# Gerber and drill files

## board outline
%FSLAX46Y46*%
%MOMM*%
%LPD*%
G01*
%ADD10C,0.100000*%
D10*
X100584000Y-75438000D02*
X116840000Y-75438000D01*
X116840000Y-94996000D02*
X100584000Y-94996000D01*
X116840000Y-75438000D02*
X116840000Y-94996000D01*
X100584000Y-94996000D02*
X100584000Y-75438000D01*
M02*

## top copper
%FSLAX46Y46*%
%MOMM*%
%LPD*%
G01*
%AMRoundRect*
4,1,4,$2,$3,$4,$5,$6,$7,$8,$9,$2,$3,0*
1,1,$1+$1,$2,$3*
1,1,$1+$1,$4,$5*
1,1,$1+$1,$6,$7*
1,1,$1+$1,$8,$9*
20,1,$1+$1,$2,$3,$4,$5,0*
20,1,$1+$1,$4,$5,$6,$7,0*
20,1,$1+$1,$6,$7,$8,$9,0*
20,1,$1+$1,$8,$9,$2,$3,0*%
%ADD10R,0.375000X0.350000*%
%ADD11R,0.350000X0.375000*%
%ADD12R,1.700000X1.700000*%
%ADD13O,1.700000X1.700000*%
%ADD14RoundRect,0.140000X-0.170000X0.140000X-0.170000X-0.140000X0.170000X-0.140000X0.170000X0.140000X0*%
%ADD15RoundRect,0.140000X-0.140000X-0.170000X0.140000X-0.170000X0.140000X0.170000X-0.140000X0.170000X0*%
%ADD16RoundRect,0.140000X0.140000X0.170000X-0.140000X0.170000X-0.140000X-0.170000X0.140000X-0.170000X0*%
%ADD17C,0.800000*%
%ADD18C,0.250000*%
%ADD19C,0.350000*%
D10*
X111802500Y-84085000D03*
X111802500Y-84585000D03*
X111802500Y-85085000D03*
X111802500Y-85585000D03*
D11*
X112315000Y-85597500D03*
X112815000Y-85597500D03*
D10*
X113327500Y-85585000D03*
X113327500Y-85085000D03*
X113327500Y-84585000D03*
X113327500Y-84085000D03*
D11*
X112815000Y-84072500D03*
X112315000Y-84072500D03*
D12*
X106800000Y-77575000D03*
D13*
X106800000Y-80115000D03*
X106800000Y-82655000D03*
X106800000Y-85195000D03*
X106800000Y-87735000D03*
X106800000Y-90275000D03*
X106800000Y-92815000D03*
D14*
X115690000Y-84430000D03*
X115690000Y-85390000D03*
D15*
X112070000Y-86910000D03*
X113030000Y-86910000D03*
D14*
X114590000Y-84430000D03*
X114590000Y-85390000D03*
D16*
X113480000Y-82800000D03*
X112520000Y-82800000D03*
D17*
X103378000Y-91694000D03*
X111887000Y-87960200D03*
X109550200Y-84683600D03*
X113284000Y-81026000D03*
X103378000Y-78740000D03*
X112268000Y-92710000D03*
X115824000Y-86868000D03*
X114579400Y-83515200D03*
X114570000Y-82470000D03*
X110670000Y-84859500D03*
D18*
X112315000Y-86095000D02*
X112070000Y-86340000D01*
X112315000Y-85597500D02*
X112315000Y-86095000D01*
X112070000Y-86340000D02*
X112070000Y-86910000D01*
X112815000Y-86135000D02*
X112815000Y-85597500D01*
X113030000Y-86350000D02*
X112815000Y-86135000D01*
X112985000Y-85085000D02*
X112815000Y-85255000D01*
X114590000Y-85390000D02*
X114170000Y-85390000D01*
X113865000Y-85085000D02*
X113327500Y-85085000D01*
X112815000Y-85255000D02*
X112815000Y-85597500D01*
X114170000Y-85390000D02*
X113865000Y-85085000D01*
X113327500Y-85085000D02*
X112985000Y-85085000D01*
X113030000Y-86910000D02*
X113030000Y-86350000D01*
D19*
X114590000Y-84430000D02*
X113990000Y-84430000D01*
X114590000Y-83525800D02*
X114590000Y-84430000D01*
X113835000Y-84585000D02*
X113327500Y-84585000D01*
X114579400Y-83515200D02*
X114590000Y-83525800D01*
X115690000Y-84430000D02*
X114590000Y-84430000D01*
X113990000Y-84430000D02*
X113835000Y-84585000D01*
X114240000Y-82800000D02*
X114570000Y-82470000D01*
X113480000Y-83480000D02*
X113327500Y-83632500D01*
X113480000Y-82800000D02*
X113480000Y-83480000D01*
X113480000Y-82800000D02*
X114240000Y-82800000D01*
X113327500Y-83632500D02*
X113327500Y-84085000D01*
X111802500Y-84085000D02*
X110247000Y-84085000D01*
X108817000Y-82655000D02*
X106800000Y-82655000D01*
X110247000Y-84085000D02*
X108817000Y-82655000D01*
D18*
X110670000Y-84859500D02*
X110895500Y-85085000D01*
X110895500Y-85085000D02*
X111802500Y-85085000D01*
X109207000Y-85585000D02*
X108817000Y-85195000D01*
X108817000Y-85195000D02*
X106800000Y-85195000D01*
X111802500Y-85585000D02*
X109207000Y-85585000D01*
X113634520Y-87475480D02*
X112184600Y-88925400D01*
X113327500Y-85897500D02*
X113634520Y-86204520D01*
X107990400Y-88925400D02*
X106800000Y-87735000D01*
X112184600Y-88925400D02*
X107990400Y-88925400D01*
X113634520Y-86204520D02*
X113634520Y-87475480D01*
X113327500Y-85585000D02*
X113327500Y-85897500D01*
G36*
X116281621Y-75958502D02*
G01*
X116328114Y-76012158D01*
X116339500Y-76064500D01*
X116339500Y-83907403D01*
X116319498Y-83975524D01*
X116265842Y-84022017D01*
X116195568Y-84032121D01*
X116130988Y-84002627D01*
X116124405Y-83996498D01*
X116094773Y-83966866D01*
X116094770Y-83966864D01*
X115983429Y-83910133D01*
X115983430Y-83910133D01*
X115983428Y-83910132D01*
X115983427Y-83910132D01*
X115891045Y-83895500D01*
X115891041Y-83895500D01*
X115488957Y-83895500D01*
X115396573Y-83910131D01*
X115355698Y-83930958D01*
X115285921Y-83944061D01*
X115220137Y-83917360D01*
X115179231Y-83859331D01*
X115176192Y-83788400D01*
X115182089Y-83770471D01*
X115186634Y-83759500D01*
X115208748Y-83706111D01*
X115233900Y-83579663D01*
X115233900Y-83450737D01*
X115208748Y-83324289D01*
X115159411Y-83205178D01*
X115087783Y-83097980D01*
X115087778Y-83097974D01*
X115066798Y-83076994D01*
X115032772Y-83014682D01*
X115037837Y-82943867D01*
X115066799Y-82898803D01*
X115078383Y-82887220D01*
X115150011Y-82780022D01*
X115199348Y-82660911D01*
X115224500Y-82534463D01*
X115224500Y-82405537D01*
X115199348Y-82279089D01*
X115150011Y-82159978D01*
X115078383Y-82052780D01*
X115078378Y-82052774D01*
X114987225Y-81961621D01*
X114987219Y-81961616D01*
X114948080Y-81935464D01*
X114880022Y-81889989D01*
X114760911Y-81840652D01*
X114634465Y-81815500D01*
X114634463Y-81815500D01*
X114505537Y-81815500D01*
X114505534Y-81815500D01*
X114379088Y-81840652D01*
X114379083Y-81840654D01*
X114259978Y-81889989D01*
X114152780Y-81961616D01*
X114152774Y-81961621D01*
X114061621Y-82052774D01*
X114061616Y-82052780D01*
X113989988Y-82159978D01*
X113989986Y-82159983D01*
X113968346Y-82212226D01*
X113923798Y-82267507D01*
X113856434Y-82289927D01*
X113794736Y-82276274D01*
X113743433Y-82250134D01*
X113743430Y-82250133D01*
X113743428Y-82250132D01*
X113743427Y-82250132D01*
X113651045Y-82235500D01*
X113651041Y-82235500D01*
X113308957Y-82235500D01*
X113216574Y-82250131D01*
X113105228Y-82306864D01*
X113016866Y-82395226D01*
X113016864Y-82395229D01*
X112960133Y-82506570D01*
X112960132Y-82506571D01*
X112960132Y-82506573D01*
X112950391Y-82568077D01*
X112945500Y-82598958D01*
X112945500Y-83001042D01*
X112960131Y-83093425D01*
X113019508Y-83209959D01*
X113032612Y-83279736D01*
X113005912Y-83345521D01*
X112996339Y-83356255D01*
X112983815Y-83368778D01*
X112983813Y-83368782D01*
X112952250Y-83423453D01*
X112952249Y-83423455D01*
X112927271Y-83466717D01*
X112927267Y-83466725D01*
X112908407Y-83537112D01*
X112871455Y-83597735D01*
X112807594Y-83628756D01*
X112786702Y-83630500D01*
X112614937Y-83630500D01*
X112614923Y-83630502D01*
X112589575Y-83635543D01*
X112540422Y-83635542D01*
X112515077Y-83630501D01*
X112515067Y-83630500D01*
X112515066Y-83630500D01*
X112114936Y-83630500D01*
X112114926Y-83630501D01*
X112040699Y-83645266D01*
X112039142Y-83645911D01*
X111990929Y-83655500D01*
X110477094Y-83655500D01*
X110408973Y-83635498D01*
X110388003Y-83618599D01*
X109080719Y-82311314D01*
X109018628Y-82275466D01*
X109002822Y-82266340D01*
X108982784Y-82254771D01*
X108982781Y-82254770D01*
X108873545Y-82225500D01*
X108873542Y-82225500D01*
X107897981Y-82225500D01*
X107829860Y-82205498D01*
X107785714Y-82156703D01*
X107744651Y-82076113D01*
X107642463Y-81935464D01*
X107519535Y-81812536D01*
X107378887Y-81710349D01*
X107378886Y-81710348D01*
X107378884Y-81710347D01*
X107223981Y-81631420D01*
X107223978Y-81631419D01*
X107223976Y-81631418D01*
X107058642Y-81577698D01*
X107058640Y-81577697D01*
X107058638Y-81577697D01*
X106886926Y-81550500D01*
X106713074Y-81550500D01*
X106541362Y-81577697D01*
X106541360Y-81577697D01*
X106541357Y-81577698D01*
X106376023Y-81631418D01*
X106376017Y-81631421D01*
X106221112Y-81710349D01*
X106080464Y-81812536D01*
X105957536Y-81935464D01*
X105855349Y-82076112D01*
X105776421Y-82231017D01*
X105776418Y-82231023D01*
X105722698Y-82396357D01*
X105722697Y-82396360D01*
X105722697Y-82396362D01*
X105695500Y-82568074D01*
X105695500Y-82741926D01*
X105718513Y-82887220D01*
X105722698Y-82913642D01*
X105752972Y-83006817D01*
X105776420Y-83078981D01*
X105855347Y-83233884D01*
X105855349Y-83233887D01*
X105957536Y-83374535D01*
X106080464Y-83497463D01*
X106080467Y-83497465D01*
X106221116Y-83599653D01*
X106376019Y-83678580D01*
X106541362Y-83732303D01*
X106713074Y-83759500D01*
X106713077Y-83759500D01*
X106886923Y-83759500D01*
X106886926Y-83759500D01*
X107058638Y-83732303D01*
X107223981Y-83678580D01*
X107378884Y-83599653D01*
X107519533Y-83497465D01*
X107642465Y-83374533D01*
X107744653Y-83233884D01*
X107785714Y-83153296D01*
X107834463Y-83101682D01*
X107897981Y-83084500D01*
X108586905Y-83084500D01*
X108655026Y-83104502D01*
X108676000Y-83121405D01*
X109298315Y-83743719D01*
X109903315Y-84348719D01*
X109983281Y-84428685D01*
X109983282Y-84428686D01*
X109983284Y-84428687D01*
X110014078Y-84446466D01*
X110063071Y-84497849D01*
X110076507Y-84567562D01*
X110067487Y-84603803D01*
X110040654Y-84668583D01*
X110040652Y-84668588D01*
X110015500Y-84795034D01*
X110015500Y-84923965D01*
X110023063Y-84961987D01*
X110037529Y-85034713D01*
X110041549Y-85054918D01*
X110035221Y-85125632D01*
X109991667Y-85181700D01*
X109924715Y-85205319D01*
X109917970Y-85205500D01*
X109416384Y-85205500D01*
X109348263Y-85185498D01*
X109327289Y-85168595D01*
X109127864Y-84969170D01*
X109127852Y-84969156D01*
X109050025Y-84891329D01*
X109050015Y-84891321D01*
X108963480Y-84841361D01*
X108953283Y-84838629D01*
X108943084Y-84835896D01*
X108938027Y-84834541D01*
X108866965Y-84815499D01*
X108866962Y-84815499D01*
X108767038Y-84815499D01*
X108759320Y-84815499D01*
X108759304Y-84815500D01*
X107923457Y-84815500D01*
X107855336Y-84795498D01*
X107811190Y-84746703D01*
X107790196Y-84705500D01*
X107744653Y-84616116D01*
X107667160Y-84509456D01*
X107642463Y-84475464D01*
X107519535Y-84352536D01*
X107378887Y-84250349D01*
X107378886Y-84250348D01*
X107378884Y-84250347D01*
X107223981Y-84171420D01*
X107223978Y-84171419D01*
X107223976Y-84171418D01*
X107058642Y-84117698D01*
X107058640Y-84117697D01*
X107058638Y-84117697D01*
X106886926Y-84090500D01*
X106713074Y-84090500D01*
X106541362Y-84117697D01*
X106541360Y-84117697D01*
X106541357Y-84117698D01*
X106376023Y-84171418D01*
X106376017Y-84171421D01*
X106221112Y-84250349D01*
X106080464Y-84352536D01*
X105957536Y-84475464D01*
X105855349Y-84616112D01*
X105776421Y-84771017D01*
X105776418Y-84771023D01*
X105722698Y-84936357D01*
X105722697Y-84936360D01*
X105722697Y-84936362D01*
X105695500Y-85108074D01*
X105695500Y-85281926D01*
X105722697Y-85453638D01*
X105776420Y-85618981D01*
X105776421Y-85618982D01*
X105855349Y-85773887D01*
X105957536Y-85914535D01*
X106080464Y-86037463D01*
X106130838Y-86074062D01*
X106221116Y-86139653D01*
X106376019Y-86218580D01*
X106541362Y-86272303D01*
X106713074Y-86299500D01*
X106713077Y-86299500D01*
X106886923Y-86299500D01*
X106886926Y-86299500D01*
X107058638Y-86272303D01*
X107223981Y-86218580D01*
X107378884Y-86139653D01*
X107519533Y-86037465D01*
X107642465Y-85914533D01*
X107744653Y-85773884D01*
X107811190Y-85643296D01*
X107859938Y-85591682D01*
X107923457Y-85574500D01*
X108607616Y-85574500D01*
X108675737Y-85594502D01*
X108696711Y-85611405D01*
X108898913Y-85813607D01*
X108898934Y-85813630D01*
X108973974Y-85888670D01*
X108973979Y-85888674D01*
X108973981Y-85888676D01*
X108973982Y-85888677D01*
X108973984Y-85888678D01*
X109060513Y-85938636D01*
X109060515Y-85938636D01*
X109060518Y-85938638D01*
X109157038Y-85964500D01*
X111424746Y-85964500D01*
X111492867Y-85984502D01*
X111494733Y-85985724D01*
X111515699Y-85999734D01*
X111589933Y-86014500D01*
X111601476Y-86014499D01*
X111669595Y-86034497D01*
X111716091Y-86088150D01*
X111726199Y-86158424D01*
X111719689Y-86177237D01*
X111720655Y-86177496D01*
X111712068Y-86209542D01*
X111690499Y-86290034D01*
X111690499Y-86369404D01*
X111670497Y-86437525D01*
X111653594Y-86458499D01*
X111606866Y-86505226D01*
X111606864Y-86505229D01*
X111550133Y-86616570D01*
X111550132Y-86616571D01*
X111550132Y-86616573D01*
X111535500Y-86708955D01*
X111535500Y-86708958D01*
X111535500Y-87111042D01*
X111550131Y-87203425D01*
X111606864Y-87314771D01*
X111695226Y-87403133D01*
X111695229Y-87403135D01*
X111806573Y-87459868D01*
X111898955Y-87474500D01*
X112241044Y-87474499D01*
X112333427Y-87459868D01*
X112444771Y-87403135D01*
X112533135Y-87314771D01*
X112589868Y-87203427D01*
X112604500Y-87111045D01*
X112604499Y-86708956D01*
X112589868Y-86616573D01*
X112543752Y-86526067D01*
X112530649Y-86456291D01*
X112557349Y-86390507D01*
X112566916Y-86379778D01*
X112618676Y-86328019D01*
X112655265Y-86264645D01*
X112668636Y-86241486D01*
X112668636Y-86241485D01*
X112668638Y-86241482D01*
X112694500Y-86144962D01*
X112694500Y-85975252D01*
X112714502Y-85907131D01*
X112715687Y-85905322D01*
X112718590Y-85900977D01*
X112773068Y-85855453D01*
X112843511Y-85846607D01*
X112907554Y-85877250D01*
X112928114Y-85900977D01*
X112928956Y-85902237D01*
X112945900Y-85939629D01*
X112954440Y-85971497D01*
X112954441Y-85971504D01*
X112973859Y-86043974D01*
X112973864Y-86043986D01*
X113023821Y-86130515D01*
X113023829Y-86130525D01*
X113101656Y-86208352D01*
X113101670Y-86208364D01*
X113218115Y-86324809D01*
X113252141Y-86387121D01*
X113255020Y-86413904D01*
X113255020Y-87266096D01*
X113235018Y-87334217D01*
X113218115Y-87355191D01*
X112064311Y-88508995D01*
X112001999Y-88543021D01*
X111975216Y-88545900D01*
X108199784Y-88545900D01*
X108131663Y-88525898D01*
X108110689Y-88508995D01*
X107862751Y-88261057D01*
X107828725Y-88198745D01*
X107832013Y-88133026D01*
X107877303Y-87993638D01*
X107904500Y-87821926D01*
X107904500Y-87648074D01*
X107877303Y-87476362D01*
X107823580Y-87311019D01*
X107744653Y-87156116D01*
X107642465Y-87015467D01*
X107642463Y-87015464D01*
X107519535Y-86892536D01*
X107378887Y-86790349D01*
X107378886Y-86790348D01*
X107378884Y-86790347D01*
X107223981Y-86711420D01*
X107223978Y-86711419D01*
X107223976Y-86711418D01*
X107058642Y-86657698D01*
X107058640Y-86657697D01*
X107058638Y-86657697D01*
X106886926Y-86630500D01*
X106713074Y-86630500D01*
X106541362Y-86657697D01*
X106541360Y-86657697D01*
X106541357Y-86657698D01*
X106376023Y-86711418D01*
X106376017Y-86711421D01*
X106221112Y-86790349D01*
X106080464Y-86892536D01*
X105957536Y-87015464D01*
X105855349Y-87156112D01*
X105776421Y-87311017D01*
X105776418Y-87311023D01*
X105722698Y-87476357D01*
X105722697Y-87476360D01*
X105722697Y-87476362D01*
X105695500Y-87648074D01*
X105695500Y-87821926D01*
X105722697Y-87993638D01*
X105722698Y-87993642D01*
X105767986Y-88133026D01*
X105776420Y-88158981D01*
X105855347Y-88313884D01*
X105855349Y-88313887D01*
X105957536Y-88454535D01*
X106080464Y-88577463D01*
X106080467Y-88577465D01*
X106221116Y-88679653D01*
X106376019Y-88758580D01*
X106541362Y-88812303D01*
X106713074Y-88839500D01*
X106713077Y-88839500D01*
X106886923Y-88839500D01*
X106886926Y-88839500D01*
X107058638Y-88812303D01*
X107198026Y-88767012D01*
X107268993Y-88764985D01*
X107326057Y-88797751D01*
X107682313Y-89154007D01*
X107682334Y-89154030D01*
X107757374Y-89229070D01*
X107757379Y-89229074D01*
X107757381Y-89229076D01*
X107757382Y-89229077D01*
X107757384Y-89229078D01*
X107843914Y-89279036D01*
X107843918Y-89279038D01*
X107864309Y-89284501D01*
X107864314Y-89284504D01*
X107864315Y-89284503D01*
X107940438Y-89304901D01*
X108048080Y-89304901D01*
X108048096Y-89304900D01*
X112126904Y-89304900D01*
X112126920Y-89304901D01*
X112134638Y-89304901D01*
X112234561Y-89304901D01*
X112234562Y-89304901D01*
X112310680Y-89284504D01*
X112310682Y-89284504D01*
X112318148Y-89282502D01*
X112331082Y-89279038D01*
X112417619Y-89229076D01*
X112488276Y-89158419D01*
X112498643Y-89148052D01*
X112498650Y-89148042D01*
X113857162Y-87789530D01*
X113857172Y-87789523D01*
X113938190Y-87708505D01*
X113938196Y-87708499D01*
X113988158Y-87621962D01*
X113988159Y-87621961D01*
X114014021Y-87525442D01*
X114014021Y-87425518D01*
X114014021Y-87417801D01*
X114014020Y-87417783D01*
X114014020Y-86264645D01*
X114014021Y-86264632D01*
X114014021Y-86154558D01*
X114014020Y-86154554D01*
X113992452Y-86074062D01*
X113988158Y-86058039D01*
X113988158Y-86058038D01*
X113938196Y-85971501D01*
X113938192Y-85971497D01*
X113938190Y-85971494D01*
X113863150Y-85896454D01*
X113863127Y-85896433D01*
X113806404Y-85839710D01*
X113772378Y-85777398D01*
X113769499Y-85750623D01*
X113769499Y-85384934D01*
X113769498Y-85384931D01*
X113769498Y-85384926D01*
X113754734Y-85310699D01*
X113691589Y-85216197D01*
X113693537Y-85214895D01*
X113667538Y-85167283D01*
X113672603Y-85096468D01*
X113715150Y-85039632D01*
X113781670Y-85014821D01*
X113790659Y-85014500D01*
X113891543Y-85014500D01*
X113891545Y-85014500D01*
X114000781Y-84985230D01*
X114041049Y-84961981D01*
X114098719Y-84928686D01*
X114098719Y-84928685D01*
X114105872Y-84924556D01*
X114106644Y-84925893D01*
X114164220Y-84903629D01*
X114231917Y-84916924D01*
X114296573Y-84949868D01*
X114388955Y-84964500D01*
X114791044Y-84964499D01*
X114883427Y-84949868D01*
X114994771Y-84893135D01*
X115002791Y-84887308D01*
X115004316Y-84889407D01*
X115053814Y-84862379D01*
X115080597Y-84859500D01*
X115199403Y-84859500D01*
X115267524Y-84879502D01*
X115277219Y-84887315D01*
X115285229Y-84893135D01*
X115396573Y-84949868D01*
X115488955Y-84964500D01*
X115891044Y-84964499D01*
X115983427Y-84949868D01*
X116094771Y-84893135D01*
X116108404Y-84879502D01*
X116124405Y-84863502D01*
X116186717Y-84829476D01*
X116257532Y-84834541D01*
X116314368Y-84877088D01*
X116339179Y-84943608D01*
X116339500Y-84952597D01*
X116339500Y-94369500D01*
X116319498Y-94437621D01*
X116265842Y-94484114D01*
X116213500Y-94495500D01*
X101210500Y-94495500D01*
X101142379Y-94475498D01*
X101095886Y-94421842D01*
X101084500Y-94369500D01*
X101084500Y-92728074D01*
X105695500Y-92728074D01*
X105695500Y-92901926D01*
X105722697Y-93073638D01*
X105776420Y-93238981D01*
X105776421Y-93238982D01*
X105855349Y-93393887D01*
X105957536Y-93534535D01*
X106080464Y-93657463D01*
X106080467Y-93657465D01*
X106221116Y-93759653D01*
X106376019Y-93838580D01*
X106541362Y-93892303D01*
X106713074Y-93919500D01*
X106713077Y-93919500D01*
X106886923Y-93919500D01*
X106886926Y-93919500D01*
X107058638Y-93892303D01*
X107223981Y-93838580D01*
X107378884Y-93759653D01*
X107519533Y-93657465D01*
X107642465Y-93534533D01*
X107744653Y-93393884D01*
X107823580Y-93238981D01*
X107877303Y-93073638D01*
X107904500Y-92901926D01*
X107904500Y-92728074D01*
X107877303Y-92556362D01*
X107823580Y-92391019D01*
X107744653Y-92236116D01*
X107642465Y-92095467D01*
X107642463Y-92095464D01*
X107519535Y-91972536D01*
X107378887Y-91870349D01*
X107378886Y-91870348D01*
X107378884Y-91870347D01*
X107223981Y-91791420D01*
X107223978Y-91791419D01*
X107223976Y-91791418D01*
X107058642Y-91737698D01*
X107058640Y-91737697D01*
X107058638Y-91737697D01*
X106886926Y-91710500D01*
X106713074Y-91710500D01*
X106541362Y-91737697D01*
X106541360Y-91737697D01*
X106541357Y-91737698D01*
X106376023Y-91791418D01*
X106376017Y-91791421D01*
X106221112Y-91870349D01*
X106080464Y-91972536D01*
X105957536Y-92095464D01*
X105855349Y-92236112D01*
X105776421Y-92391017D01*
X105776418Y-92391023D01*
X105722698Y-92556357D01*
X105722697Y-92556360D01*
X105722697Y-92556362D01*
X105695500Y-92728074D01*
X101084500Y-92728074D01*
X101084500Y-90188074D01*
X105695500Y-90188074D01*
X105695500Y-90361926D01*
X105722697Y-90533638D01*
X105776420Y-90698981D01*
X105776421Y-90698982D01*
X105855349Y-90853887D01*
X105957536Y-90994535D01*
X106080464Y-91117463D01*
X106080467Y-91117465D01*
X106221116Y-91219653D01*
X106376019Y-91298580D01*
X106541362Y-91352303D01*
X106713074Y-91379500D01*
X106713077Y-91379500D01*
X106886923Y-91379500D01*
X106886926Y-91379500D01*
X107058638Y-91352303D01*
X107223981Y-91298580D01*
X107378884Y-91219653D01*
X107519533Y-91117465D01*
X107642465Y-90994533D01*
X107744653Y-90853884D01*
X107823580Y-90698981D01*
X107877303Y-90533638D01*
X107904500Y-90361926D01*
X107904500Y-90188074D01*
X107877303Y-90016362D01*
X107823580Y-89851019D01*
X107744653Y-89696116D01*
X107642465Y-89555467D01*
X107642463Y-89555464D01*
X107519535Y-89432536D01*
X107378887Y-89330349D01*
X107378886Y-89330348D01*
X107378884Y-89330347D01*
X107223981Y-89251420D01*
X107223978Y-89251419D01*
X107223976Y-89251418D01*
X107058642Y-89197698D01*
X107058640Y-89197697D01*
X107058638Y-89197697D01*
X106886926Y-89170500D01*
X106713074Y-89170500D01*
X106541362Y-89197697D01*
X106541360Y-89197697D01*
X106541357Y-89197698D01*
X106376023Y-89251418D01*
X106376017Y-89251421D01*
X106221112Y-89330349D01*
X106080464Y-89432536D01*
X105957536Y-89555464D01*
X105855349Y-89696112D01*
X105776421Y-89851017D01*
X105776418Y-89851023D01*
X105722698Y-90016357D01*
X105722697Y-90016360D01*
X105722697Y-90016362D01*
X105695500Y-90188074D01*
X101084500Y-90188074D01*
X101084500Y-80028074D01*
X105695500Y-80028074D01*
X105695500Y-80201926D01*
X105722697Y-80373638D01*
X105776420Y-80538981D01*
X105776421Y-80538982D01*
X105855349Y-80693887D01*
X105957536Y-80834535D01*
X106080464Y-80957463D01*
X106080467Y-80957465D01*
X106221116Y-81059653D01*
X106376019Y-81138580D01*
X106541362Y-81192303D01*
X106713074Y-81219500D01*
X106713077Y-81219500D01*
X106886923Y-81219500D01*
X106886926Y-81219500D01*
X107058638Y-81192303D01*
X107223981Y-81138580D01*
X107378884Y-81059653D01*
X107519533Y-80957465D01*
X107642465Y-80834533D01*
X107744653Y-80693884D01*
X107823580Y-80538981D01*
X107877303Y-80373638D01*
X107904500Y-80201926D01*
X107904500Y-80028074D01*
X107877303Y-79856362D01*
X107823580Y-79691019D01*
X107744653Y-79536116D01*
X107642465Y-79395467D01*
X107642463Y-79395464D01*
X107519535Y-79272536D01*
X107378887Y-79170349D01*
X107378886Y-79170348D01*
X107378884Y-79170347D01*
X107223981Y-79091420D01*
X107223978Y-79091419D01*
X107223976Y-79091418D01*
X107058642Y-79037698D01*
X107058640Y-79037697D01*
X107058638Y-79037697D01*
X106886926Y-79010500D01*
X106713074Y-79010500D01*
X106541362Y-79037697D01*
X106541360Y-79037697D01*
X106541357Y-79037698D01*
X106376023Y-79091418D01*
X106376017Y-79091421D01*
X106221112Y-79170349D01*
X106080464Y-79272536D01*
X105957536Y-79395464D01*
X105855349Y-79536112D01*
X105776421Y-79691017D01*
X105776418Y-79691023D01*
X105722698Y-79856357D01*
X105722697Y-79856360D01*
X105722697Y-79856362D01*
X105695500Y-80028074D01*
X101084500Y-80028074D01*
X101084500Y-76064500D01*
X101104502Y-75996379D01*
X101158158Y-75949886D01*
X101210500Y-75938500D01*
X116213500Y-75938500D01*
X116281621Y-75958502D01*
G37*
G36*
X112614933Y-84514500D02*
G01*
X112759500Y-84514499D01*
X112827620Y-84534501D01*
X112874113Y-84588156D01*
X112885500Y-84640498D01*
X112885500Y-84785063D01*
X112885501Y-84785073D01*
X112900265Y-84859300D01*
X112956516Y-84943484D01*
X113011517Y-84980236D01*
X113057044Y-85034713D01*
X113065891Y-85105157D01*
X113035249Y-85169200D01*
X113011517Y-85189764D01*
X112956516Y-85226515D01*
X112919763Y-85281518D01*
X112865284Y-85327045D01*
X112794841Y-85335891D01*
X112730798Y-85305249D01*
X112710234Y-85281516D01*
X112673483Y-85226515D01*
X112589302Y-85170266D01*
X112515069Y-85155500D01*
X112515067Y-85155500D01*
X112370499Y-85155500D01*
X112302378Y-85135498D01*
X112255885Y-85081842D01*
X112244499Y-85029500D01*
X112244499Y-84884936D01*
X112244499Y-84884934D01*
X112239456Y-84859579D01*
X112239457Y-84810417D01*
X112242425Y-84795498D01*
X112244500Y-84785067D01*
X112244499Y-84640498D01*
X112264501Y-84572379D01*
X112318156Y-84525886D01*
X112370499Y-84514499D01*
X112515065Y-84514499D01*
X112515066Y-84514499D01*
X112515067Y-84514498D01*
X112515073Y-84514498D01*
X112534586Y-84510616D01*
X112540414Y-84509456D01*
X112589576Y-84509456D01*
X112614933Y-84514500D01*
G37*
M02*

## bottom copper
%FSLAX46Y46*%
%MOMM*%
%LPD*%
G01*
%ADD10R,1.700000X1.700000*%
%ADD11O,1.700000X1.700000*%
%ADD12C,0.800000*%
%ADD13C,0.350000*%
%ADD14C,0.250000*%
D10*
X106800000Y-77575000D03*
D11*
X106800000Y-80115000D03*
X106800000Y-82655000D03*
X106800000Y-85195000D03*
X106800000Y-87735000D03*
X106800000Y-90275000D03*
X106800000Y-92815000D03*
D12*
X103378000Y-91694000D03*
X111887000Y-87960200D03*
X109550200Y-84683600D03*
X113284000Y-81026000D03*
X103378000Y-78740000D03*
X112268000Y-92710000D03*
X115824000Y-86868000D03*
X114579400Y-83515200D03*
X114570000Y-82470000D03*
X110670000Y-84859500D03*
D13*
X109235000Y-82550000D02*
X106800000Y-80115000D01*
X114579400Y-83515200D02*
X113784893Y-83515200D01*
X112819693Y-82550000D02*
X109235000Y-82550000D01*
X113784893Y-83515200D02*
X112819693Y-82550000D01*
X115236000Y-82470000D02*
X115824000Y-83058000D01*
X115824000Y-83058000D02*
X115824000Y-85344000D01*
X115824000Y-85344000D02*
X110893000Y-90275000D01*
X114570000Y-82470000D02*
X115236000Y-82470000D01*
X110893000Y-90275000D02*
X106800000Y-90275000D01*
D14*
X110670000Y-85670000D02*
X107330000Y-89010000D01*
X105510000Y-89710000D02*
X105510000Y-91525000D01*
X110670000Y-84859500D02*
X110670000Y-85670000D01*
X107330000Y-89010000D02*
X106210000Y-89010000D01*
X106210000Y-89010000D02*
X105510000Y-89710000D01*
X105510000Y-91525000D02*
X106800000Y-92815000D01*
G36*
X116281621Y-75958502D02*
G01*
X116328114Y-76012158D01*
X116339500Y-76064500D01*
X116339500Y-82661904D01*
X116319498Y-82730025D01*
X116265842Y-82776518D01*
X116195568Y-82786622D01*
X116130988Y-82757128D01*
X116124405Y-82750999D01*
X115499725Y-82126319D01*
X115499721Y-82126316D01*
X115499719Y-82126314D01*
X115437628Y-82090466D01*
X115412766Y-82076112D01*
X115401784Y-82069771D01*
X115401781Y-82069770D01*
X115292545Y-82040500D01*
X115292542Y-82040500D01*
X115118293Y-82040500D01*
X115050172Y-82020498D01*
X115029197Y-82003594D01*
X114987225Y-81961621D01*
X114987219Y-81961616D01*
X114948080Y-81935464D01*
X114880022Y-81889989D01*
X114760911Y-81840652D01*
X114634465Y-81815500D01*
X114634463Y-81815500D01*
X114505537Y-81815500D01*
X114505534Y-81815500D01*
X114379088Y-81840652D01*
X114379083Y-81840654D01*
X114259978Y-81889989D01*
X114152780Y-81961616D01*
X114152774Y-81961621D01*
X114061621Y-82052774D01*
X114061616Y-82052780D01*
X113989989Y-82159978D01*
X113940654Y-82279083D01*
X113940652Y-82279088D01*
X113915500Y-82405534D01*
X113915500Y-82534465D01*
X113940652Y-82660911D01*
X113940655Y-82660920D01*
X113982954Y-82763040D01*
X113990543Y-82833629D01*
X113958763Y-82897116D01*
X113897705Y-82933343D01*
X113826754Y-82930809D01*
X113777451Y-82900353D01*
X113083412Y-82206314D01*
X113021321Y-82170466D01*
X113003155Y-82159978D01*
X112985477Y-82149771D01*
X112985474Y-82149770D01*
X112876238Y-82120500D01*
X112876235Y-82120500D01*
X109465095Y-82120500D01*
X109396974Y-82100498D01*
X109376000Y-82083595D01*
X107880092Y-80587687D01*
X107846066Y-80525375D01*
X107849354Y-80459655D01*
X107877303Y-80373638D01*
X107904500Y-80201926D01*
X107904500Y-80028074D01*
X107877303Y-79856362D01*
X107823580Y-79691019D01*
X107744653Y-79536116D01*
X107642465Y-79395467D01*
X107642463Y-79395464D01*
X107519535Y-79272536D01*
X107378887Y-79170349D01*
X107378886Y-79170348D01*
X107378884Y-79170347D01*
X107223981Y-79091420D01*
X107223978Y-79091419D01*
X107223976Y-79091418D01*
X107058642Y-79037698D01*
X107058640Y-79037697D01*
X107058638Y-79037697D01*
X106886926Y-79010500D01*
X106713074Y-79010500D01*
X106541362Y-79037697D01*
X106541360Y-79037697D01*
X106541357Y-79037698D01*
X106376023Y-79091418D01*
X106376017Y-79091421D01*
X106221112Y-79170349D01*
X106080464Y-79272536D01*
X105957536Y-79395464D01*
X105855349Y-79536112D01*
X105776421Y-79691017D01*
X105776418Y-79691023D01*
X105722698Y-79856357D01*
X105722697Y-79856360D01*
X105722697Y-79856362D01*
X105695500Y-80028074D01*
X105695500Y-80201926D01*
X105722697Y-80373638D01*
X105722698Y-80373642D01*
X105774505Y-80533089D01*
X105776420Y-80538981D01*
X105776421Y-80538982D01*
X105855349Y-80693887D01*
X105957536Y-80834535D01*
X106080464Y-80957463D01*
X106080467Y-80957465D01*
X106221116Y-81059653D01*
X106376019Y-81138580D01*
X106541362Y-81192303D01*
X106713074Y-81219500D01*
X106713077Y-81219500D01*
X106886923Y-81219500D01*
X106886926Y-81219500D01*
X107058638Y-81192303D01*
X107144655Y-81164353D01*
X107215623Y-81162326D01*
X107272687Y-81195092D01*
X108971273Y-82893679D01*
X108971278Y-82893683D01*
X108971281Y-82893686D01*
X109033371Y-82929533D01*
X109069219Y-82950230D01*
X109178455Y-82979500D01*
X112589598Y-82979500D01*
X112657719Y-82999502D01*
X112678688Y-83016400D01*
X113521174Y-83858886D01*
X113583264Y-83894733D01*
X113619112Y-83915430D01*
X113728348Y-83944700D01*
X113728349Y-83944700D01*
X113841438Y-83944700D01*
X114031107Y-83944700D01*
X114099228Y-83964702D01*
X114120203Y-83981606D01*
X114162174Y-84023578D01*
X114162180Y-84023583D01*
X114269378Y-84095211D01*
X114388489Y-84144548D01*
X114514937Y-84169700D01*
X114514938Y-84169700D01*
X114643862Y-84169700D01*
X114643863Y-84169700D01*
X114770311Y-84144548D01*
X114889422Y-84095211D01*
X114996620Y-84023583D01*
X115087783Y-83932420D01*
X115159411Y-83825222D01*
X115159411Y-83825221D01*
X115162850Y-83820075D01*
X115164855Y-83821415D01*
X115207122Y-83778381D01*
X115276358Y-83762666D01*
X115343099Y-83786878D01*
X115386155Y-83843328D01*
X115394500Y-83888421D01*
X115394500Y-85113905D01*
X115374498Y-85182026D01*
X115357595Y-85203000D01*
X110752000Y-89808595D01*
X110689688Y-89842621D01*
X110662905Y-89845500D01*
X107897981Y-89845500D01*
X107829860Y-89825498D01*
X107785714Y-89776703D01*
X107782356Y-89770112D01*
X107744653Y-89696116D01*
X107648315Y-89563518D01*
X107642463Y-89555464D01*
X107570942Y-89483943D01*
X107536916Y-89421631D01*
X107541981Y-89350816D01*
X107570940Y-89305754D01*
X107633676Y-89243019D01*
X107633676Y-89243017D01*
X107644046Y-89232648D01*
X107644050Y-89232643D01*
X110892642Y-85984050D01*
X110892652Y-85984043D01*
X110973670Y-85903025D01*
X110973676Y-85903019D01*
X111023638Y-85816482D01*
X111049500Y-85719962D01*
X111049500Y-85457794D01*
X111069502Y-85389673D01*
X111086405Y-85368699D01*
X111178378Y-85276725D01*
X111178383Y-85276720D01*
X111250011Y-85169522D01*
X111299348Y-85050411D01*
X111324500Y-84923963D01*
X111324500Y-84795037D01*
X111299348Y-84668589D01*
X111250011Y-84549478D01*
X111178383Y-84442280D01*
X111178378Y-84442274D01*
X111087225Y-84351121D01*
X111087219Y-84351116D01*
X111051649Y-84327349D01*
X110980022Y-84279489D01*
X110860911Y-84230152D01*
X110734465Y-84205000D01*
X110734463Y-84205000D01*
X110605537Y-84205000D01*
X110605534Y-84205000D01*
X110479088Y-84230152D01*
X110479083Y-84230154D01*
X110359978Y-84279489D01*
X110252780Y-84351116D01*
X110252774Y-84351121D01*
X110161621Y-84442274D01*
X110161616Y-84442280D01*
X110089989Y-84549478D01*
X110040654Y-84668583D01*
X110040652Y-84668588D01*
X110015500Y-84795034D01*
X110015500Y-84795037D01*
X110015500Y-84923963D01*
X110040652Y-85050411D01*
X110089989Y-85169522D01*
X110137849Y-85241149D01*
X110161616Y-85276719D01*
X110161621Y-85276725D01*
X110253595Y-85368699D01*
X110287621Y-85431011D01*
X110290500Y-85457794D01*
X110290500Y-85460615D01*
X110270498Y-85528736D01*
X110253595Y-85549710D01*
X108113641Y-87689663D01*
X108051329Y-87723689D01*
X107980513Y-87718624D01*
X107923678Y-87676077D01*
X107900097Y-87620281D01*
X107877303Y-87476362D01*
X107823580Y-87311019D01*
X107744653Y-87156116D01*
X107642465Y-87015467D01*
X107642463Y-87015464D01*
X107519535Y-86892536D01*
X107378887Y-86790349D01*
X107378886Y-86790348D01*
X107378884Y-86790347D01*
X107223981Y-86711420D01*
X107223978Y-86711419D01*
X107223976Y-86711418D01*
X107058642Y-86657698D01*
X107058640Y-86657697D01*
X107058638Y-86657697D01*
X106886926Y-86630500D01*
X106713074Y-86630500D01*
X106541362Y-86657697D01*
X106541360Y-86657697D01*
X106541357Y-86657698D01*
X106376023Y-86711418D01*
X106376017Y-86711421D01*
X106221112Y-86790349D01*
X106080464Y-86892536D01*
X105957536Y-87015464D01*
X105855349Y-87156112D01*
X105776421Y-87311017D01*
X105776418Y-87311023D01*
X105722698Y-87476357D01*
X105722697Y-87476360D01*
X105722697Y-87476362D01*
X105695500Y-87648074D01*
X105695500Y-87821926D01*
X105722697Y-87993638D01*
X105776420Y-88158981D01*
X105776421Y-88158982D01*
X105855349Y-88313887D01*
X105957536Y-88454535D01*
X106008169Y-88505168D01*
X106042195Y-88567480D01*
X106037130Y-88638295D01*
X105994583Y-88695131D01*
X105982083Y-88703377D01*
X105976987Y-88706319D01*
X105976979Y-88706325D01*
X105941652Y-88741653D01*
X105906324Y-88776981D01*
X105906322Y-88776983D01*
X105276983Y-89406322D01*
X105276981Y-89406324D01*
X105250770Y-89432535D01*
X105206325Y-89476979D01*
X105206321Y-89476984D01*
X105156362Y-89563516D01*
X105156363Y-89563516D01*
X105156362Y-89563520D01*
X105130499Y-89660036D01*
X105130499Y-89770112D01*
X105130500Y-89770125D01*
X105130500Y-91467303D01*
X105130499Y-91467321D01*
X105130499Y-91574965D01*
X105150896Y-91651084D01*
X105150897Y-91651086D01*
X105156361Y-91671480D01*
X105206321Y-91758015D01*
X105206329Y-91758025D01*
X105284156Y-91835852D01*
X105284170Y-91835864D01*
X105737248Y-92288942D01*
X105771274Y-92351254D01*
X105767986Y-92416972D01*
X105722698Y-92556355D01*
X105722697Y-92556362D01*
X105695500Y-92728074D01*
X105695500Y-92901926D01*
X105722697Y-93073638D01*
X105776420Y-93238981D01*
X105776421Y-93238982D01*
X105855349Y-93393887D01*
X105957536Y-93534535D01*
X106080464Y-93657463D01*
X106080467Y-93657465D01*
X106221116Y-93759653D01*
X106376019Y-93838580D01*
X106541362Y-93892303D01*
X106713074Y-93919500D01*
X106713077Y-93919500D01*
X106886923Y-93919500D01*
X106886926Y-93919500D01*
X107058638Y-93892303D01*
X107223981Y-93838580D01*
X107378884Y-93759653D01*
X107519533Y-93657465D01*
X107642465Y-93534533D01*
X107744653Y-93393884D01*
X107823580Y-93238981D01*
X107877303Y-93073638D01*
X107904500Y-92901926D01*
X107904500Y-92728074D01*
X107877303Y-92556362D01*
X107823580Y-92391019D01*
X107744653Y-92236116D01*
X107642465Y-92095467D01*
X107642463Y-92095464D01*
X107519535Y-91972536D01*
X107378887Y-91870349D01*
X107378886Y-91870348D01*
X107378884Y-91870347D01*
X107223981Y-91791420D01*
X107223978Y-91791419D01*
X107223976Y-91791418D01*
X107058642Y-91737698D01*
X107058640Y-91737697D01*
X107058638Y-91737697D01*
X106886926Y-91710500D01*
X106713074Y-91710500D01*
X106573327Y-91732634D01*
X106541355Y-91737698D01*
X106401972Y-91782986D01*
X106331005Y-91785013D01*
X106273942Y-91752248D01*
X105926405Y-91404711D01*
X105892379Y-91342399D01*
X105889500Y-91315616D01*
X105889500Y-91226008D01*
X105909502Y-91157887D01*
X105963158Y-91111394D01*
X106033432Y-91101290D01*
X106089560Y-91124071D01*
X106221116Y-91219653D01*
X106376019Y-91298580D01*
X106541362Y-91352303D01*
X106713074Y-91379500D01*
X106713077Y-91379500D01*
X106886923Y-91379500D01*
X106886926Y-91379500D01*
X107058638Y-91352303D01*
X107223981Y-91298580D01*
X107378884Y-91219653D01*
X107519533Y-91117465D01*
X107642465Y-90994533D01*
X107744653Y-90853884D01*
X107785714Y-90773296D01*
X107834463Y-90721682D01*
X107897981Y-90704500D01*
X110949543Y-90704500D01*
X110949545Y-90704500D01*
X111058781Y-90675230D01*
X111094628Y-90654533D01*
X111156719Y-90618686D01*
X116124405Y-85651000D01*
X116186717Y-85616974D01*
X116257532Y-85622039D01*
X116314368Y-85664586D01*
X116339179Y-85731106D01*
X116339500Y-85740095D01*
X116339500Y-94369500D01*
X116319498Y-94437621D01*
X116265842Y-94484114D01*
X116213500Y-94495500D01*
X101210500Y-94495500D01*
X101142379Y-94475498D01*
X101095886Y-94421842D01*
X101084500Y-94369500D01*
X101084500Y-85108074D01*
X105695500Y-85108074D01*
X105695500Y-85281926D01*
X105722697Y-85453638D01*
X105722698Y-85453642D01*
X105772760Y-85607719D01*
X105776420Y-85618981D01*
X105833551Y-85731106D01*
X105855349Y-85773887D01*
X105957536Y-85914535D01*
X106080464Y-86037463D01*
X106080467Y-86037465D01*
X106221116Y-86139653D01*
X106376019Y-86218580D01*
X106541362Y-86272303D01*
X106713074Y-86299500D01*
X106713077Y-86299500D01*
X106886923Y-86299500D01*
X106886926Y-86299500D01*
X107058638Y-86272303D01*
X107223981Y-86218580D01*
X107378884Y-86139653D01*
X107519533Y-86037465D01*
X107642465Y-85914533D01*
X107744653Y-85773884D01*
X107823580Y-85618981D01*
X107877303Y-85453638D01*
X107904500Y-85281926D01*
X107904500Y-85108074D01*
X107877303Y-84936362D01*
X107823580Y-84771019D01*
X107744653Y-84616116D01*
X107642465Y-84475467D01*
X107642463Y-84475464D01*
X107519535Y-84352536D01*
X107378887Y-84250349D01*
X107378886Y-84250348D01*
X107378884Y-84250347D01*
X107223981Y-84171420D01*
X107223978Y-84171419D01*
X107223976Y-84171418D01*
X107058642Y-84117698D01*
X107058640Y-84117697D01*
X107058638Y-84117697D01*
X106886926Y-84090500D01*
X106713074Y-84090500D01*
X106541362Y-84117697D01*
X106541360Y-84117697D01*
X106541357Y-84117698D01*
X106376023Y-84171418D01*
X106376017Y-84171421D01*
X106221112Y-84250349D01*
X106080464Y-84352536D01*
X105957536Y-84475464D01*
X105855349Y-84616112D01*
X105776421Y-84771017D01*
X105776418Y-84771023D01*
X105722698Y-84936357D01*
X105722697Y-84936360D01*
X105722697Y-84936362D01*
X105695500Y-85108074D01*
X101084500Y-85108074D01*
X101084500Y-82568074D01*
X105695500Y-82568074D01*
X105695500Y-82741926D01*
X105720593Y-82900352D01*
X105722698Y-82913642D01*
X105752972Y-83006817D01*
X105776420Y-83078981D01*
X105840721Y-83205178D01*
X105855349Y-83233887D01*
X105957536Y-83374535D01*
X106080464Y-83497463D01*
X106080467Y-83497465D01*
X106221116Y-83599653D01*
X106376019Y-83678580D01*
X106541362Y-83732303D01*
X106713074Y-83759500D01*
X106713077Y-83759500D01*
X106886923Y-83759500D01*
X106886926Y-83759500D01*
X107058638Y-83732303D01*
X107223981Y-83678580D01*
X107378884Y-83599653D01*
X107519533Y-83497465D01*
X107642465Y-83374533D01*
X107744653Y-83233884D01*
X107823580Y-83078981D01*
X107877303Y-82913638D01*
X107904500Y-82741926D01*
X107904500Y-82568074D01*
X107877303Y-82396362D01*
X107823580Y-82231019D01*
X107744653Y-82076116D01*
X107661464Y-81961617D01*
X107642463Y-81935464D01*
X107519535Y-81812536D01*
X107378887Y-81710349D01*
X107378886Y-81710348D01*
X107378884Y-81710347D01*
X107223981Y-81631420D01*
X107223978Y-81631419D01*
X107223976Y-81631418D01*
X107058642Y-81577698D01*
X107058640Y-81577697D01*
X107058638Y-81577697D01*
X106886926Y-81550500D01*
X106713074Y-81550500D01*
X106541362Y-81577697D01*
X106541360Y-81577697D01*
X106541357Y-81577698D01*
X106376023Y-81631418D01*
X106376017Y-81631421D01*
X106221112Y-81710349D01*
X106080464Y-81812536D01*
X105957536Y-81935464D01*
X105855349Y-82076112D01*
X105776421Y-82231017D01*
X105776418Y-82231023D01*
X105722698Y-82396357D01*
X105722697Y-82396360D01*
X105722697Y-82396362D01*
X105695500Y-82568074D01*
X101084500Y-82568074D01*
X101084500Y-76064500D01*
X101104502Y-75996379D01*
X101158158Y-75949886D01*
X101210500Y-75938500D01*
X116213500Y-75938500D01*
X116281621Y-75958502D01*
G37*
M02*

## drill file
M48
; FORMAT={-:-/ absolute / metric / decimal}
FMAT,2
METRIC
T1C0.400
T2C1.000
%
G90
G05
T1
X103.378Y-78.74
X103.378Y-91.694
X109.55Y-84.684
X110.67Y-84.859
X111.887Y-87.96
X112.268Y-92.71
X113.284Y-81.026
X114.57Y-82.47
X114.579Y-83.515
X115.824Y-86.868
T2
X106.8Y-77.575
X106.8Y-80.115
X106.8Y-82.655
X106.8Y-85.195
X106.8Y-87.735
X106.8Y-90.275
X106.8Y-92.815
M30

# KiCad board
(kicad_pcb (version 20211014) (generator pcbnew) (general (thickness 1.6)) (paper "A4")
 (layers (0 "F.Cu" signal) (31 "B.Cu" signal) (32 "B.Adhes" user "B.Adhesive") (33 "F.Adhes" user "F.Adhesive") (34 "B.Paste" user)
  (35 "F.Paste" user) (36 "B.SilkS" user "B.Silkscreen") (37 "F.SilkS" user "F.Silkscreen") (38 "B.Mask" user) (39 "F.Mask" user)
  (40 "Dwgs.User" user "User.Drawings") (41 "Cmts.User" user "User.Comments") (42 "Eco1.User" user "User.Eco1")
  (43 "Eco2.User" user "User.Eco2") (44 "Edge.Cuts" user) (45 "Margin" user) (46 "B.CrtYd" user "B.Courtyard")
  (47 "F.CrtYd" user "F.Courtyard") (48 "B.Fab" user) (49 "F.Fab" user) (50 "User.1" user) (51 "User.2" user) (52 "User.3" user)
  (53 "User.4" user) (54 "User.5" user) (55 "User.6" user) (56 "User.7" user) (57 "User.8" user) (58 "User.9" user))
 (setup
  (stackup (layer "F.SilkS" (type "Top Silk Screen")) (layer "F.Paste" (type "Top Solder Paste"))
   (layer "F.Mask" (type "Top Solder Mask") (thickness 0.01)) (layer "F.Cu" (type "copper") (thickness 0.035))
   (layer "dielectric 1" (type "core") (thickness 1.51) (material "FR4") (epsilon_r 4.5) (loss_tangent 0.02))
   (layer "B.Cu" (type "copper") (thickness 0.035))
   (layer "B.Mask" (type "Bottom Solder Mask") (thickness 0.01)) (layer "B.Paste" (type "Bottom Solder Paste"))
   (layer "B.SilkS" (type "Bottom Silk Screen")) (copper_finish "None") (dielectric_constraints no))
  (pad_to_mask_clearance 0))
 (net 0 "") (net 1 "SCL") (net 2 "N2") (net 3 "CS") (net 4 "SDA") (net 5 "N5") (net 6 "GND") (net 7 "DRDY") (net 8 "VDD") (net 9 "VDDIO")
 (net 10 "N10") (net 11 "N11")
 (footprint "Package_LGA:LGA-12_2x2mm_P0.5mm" (layer "F.Cu") (at 112.565 84.835)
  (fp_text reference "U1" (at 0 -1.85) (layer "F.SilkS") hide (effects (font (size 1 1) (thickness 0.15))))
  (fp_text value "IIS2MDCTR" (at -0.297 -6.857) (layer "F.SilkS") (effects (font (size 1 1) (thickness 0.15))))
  (pad "1" smd rect (at -0.7625 -0.75) (size 0.375 0.35) (layers "F.Cu" "F.Paste" "F.Mask") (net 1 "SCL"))
  (pad "2" smd rect (at -0.7625 -0.25) (size 0.375 0.35) (layers "F.Cu" "F.Paste" "F.Mask") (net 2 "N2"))
  (pad "3" smd rect (at -0.7625 0.25) (size 0.375 0.35) (layers "F.Cu" "F.Paste" "F.Mask") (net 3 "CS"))
  (pad "4" smd rect (at -0.7625 0.75) (size 0.375 0.35) (layers "F.Cu" "F.Paste" "F.Mask") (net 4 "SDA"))
  (pad "5" smd rect (at -0.25 0.7625 90) (size 0.375 0.35) (layers "F.Cu" "F.Paste" "F.Mask") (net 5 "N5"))
  (pad "6" smd rect (at 0.25 0.7625 90) (size 0.375 0.35) (layers "F.Cu" "F.Paste" "F.Mask") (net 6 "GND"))
  (pad "7" smd rect (at 0.7625 0.75) (size 0.375 0.35) (layers "F.Cu" "F.Paste" "F.Mask") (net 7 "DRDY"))
  (pad "8" smd rect (at 0.7625 0.25) (size 0.375 0.35) (layers "F.Cu" "F.Paste" "F.Mask") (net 6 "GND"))
  (pad "9" smd rect (at 0.7625 -0.25) (size 0.375 0.35) (layers "F.Cu" "F.Paste" "F.Mask") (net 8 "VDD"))
  (pad "10" smd rect (at 0.7625 -0.75) (size 0.375 0.35) (layers "F.Cu" "F.Paste" "F.Mask") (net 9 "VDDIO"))
  (pad "11" smd rect (at 0.25 -0.7625 90) (size 0.375 0.35) (layers "F.Cu" "F.Paste" "F.Mask") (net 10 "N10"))
  (pad "12" smd rect (at -0.25 -0.7625 90) (size 0.375 0.35) (layers "F.Cu" "F.Paste" "F.Mask") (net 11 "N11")))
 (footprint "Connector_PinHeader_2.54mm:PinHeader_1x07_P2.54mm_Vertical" (layer "F.Cu") (at 106.8 77.575)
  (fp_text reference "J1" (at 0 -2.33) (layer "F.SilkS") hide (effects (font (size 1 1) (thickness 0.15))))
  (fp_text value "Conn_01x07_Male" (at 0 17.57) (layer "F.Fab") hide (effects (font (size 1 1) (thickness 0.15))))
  (pad "1" thru_hole rect (at 0 0) (size 1.7 1.7) (drill 1) (layers *.Cu *.Mask) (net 6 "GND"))
  (pad "2" thru_hole oval (at 0 2.54) (size 1.7 1.7) (drill 1) (layers *.Cu *.Mask) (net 8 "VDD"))
  (pad "3" thru_hole oval (at 0 5.08) (size 1.7 1.7) (drill 1) (layers *.Cu *.Mask) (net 1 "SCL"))
  (pad "4" thru_hole oval (at 0 7.62) (size 1.7 1.7) (drill 1) (layers *.Cu *.Mask) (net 4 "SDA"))
  (pad "5" thru_hole oval (at 0 10.16) (size 1.7 1.7) (drill 1) (layers *.Cu *.Mask) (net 7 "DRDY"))
  (pad "6" thru_hole oval (at 0 12.7) (size 1.7 1.7) (drill 1) (layers *.Cu *.Mask) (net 9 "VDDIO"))
  (pad "7" thru_hole oval (at 0 15.24) (size 1.7 1.7) (drill 1) (layers *.Cu *.Mask) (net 3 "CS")))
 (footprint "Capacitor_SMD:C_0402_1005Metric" (layer "F.Cu") (at 115.69 84.91 -90)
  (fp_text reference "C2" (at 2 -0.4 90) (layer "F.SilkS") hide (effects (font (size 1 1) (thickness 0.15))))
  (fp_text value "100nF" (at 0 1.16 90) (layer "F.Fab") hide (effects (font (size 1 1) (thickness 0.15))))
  (pad "1" smd roundrect (at -0.48 0 270) (size 0.56 0.62) (layers "F.Cu" "F.Paste" "F.Mask") (roundrect_rratio 0.25) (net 8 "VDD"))
  (pad "2" smd roundrect (at 0.48 0 270) (size 0.56 0.62) (layers "F.Cu" "F.Paste" "F.Mask") (roundrect_rratio 0.25) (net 6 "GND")))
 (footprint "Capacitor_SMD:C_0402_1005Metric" (layer "F.Cu") (at 112.55 86.91)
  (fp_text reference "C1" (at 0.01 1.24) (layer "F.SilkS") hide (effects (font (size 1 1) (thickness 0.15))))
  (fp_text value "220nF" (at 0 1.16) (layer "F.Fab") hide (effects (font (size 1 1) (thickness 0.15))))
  (pad "1" smd roundrect (at -0.48 0) (size 0.56 0.62) (layers "F.Cu" "F.Paste" "F.Mask") (roundrect_rratio 0.25) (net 5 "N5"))
  (pad "2" smd roundrect (at 0.48 0) (size 0.56 0.62) (layers "F.Cu" "F.Paste" "F.Mask") (roundrect_rratio 0.25) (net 6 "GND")))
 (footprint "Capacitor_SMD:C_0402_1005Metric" (layer "F.Cu") (at 114.59 84.91 -90)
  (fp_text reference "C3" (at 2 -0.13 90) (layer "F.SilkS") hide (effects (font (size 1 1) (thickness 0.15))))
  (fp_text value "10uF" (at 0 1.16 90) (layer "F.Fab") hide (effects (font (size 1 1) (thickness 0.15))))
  (pad "1" smd roundrect (at -0.48 0 270) (size 0.56 0.62) (layers "F.Cu" "F.Paste" "F.Mask") (roundrect_rratio 0.25) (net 8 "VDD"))
  (pad "2" smd roundrect (at 0.48 0 270) (size 0.56 0.62) (layers "F.Cu" "F.Paste" "F.Mask") (roundrect_rratio 0.25) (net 6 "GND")))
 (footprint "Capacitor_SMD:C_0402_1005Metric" (layer "F.Cu") (at 113 82.8 180)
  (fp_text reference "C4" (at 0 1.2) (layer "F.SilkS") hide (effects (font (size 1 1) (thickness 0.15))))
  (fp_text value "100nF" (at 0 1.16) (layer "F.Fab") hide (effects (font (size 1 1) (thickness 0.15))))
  (pad "1" smd roundrect (at -0.48 0 180) (size 0.56 0.62) (layers "F.Cu" "F.Paste" "F.Mask") (roundrect_rratio 0.25) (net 9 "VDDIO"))
  (pad "2" smd roundrect (at 0.48 0 180) (size 0.56 0.62) (layers "F.Cu" "F.Paste" "F.Mask") (roundrect_rratio 0.25) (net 6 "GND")))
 (gr_line (start 100.584 75.438) (end 116.84 75.438) (layer "Edge.Cuts") (width 0.1))
 (gr_line (start 116.84 94.996) (end 100.584 94.996) (layer "Edge.Cuts") (width 0.1))
 (gr_line (start 116.84 75.438) (end 116.84 94.996) (layer "Edge.Cuts") (width 0.1))
 (gr_line (start 100.584 94.996) (end 100.584 75.438) (layer "Edge.Cuts") (width 0.1))
 (segment (start 112.315 86.095) (end 112.07 86.34) (width 0.25) (layer "F.Cu") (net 5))
 (segment (start 112.315 85.5975) (end 112.315 86.095) (width 0.25) (layer "F.Cu") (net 5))
 (segment (start 112.07 86.34) (end 112.07 86.91) (width 0.25) (layer "F.Cu") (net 5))
 (segment (start 112.815 86.135) (end 112.815 85.5975) (width 0.25) (layer "F.Cu") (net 6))
 (segment (start 113.03 86.35) (end 112.815 86.135) (width 0.25) (layer "F.Cu") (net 6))
 (segment (start 112.985 85.085) (end 112.815 85.255) (width 0.25) (layer "F.Cu") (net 6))
 (segment (start 114.59 85.39) (end 114.17 85.39) (width 0.25) (layer "F.Cu") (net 6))
 (segment (start 113.865 85.085) (end 113.3275 85.085) (width 0.25) (layer "F.Cu") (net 6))
 (segment (start 112.815 85.255) (end 112.815 85.5975) (width 0.25) (layer "F.Cu") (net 6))
 (segment (start 114.17 85.39) (end 113.865 85.085) (width 0.25) (layer "F.Cu") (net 6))
 (segment (start 113.3275 85.085) (end 112.985 85.085) (width 0.25) (layer "F.Cu") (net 6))
 (segment (start 113.03 86.91) (end 113.03 86.35) (width 0.25) (layer "F.Cu") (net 6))
 (via (at 103.378 91.694) (size 0.8) (drill 0.4) (layers "F.Cu" "B.Cu") (free) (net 6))
 (via (at 111.887 87.9602) (size 0.8) (drill 0.4) (layers "F.Cu" "B.Cu") (free) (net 6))
 (via (at 109.5502 84.6836) (size 0.8) (drill 0.4) (layers "F.Cu" "B.Cu") (free) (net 6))
 (via (at 113.284 81.026) (size 0.8) (drill 0.4) (layers "F.Cu" "B.Cu") (free) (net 6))
 (via (at 103.378 78.74) (size 0.8) (drill 0.4) (layers "F.Cu" "B.Cu") (free) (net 6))
 (via (at 112.268 92.71) (size 0.8) (drill 0.4) (layers "F.Cu" "B.Cu") (free) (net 6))
 (via (at 115.824 86.868) (size 0.8) (drill 0.4) (layers "F.Cu" "B.Cu") (free) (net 6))
 (segment (start 114.59 84.43) (end 113.99 84.43) (width 0.35) (layer "F.Cu") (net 8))
 (segment (start 114.59 83.5258) (end 114.59 84.43) (width 0.35) (layer "F.Cu") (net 8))
 (segment (start 113.835 84.585) (end 113.3275 84.585) (width 0.35) (layer "F.Cu") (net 8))
 (segment (start 114.5794 83.5152) (end 114.59 83.5258) (width 0.35) (layer "F.Cu") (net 8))
 (segment (start 115.69 84.43) (end 114.59 84.43) (width 0.35) (layer "F.Cu") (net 8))
 (segment (start 113.99 84.43) (end 113.835 84.585) (width 0.35) (layer "F.Cu") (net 8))
 (via (at 114.5794 83.5152) (size 0.8) (drill 0.4) (layers "F.Cu" "B.Cu") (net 8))
 (segment (start 109.235 82.55) (end 106.8 80.115) (width 0.35) (layer "B.Cu") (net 8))
 (segment (start 114.5794 83.5152) (end 113.784893 83.5152) (width 0.35) (layer "B.Cu") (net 8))
 (segment (start 112.819693 82.55) (end 109.235 82.55) (width 0.35) (layer "B.Cu") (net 8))
 (segment (start 113.784893 83.5152) (end 112.819693 82.55) (width 0.35) (layer "B.Cu") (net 8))
 (segment (start 114.24 82.8) (end 114.57 82.47) (width 0.35) (layer "F.Cu") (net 9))
 (segment (start 113.48 83.48) (end 113.3275 83.6325) (width 0.35) (layer "F.Cu") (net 9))
 (segment (start 113.48 82.8) (end 113.48 83.48) (width 0.35) (layer "F.Cu") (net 9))
 (segment (start 113.48 82.8) (end 114.24 82.8) (width 0.35) (layer "F.Cu") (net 9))
 (segment (start 113.3275 83.6325) (end 113.3275 84.085) (width 0.35) (layer "F.Cu") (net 9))
 (via (at 114.57 82.47) (size 0.8) (drill 0.4) (layers "F.Cu" "B.Cu") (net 9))
 (segment (start 115.236 82.47) (end 115.824 83.058) (width 0.35) (layer "B.Cu") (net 9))
 (segment (start 115.824 83.058) (end 115.824 85.344) (width 0.35) (layer "B.Cu") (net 9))
 (segment (start 115.824 85.344) (end 110.893 90.275) (width 0.35) (layer "B.Cu") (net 9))
 (segment (start 114.57 82.47) (end 115.236 82.47) (width 0.35) (layer "B.Cu") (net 9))
 (segment (start 110.893 90.275) (end 106.8 90.275) (width 0.35) (layer "B.Cu") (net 9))
 (segment (start 111.8025 84.085) (end 110.247 84.085) (width 0.35) (layer "F.Cu") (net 1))
 (segment (start 108.817 82.655) (end 106.8 82.655) (width 0.35) (layer "F.Cu") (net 1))
 (segment (start 110.247 84.085) (end 108.817 82.655) (width 0.35) (layer "F.Cu") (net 1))
 (segment (start 110.67 84.8595) (end 110.8955 85.085) (width 0.25) (layer "F.Cu") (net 3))
 (segment (start 110.8955 85.085) (end 111.8025 85.085) (width 0.25) (layer "F.Cu") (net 3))
 (via (at 110.67 84.8595) (size 0.8) (drill 0.4) (layers "F.Cu" "B.Cu") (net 3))
 (segment (start 110.67 85.67) (end 107.33 89.01) (width 0.25) (layer "B.Cu") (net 3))
 (segment (start 105.51 89.71) (end 105.51 91.525) (width 0.25) (layer "B.Cu") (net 3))
 (segment (start 110.67 84.8595) (end 110.67 85.67) (width 0.25) (layer "B.Cu") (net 3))
 (segment (start 107.33 89.01) (end 106.21 89.01) (width 0.25) (layer "B.Cu") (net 3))
 (segment (start 106.21 89.01) (end 105.51 89.71) (width 0.25) (layer "B.Cu") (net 3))
 (segment (start 105.51 91.525) (end 106.8 92.815) (width 0.25) (layer "B.Cu") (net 3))
 (segment (start 109.207 85.585) (end 108.817 85.195) (width 0.25) (layer "F.Cu") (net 4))
 (segment (start 108.817 85.195) (end 106.8 85.195) (width 0.25) (layer "F.Cu") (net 4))
 (segment (start 111.8025 85.585) (end 109.207 85.585) (width 0.25) (layer "F.Cu") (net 4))
 (segment (start 113.63452 87.47548) (end 112.1846 88.9254) (width 0.25) (layer "F.Cu") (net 7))
 (segment (start 113.3275 85.8975) (end 113.63452 86.20452) (width 0.25) (layer "F.Cu") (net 7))
 (segment (start 107.9904 88.9254) (end 106.8 87.735) (width 0.25) (layer "F.Cu") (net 7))
 (segment (start 112.1846 88.9254) (end 107.9904 88.9254) (width 0.25) (layer "F.Cu") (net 7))
 (segment (start 113.63452 86.20452) (end 113.63452 87.47548) (width 0.25) (layer "F.Cu") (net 7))
 (segment (start 113.3275 85.585) (end 113.3275 85.8975) (width 0.25) (layer "F.Cu") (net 7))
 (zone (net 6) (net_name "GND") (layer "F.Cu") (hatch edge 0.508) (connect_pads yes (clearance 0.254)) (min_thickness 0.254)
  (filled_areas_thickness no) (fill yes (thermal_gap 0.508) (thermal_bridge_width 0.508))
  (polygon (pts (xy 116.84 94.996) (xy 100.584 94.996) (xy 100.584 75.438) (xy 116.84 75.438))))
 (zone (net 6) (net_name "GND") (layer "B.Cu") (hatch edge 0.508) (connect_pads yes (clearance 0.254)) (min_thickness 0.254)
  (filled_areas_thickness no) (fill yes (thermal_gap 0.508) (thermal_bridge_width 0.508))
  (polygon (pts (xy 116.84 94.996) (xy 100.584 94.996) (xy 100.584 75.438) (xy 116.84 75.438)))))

